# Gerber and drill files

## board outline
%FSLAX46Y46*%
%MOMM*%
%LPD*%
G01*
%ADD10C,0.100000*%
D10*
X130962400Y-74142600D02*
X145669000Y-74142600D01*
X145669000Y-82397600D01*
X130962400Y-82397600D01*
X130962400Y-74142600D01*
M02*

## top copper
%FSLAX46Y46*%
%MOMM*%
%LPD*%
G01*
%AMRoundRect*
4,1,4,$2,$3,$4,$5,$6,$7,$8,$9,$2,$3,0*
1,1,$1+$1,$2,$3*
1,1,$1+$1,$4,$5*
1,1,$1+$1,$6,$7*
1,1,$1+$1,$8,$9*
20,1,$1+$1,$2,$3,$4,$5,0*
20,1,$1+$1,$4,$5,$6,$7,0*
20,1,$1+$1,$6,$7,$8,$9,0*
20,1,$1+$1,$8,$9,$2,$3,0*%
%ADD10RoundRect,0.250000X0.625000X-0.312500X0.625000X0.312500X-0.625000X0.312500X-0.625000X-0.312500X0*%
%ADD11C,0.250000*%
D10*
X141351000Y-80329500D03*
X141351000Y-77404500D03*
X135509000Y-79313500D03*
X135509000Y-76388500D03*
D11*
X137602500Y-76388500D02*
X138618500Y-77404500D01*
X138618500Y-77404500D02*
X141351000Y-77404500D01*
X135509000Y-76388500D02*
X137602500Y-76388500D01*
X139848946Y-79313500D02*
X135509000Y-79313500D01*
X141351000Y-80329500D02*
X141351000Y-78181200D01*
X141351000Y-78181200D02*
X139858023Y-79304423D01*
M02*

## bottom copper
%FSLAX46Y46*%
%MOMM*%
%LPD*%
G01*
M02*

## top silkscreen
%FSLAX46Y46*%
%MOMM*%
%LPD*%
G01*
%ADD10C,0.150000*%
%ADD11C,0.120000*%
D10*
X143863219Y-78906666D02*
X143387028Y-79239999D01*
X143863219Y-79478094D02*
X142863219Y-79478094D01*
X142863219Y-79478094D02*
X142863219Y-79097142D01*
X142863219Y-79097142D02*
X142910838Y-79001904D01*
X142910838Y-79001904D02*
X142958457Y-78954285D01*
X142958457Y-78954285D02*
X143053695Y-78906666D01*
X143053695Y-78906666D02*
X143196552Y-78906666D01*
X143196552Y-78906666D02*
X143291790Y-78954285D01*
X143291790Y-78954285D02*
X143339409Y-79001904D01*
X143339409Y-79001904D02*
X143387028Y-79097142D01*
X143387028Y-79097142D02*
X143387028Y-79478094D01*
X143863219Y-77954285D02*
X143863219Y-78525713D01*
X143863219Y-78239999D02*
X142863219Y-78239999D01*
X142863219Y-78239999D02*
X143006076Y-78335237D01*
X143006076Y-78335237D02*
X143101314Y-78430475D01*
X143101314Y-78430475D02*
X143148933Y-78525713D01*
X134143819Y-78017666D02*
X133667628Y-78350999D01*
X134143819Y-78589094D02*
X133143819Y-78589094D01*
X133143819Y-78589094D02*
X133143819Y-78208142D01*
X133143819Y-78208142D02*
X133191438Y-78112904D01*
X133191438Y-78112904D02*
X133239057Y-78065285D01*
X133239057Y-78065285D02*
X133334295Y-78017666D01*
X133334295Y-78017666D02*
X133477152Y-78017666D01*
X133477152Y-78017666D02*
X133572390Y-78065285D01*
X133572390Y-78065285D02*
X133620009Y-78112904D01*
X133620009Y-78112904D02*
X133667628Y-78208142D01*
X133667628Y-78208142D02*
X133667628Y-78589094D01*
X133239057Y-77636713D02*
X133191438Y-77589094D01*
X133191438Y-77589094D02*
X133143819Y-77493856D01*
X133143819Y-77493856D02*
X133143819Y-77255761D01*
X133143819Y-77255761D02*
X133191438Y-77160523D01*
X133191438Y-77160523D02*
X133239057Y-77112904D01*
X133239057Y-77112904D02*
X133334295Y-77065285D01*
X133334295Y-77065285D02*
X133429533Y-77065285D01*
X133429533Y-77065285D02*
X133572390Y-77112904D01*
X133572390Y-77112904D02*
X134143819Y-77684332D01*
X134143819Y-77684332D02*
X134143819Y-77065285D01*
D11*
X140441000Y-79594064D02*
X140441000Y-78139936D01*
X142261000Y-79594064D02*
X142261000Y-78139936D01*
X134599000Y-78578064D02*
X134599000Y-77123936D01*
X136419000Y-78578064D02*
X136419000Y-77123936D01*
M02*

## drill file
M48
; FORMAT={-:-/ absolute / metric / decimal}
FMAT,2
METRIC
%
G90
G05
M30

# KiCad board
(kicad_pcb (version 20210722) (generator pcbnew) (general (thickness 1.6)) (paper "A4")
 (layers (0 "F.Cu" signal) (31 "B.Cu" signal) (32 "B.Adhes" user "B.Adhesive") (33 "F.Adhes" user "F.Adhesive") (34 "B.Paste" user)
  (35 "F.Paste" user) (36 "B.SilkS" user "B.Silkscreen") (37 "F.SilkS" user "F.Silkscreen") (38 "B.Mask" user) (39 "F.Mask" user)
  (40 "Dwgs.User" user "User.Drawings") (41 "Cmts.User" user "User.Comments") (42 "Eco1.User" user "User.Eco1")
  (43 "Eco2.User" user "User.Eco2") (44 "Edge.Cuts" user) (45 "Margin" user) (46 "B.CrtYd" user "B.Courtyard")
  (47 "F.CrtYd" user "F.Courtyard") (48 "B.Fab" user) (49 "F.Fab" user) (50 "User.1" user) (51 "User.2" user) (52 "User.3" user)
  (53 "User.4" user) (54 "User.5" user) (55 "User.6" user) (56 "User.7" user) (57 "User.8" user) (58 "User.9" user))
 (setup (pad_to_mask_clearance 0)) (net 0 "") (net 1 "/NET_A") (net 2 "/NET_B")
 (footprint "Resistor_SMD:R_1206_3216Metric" (layer "F.Cu") (at 141.351 78.867 90)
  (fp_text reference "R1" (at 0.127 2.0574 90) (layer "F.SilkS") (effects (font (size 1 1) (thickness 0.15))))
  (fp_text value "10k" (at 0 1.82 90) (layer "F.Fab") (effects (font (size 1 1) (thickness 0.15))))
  (fp_line (start -0.727064 -0.91) (end 0.727064 -0.91) (layer "F.SilkS") (width 0.12))
  (fp_line (start -0.727064 0.91) (end 0.727064 0.91) (layer "F.SilkS") (width 0.12))
  (pad "1" smd roundrect locked (at -1.4625 0 90) (size 1.125 1.75) (layers "F.Cu" "F.Paste" "F.Mask") (roundrect_rratio 0.222222)
   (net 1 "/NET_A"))
  (pad "2" smd roundrect locked (at 1.4625 0 90) (size 1.125 1.75) (layers "F.Cu" "F.Paste" "F.Mask") (roundrect_rratio 0.222222)
   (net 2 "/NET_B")))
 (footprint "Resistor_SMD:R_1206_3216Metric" (layer "F.Cu") (at 135.509 77.851 90)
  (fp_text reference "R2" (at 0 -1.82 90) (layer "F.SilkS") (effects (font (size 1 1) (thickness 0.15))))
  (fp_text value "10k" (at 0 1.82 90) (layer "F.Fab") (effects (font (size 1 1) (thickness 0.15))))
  (fp_line (start -0.727064 -0.91) (end 0.727064 -0.91) (layer "F.SilkS") (width 0.12))
  (fp_line (start -0.727064 0.91) (end 0.727064 0.91) (layer "F.SilkS") (width 0.12))
  (pad "1" smd roundrect locked (at -1.4625 0 90) (size 1.125 1.75) (layers "F.Cu" "F.Paste" "F.Mask") (roundrect_rratio 0.222222)
   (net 1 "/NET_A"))
  (pad "2" smd roundrect locked (at 1.4625 0 90) (size 1.125 1.75) (layers "F.Cu" "F.Paste" "F.Mask") (roundrect_rratio 0.222222)
   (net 2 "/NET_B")))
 (gr_rect (start 130.9624 74.1426) (end 145.669 82.3976) (layer "Edge.Cuts") (width 0.1) (fill none))
 (segment (start 137.6025 76.3885) (end 138.6185 77.4045) (width 0.25) (layer "F.Cu") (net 2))
 (segment (start 138.6185 77.4045) (end 141.351 77.4045) (width 0.25) (layer "F.Cu") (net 2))
 (segment (start 135.509 76.3885) (end 137.6025 76.3885) (width 0.25) (layer "F.Cu") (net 2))
 (segment (start 139.848946 79.3135) (end 135.509 79.3135) (width 0.25) (layer "F.Cu") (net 1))
 (segment (start 141.351 80.3295) (end 141.351 78.1812) (width 0.25) (layer "F.Cu") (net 1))
 (segment (start 141.351 78.1812) (end 139.858023 79.304423) (width 0.25) (layer "F.Cu") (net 1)))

